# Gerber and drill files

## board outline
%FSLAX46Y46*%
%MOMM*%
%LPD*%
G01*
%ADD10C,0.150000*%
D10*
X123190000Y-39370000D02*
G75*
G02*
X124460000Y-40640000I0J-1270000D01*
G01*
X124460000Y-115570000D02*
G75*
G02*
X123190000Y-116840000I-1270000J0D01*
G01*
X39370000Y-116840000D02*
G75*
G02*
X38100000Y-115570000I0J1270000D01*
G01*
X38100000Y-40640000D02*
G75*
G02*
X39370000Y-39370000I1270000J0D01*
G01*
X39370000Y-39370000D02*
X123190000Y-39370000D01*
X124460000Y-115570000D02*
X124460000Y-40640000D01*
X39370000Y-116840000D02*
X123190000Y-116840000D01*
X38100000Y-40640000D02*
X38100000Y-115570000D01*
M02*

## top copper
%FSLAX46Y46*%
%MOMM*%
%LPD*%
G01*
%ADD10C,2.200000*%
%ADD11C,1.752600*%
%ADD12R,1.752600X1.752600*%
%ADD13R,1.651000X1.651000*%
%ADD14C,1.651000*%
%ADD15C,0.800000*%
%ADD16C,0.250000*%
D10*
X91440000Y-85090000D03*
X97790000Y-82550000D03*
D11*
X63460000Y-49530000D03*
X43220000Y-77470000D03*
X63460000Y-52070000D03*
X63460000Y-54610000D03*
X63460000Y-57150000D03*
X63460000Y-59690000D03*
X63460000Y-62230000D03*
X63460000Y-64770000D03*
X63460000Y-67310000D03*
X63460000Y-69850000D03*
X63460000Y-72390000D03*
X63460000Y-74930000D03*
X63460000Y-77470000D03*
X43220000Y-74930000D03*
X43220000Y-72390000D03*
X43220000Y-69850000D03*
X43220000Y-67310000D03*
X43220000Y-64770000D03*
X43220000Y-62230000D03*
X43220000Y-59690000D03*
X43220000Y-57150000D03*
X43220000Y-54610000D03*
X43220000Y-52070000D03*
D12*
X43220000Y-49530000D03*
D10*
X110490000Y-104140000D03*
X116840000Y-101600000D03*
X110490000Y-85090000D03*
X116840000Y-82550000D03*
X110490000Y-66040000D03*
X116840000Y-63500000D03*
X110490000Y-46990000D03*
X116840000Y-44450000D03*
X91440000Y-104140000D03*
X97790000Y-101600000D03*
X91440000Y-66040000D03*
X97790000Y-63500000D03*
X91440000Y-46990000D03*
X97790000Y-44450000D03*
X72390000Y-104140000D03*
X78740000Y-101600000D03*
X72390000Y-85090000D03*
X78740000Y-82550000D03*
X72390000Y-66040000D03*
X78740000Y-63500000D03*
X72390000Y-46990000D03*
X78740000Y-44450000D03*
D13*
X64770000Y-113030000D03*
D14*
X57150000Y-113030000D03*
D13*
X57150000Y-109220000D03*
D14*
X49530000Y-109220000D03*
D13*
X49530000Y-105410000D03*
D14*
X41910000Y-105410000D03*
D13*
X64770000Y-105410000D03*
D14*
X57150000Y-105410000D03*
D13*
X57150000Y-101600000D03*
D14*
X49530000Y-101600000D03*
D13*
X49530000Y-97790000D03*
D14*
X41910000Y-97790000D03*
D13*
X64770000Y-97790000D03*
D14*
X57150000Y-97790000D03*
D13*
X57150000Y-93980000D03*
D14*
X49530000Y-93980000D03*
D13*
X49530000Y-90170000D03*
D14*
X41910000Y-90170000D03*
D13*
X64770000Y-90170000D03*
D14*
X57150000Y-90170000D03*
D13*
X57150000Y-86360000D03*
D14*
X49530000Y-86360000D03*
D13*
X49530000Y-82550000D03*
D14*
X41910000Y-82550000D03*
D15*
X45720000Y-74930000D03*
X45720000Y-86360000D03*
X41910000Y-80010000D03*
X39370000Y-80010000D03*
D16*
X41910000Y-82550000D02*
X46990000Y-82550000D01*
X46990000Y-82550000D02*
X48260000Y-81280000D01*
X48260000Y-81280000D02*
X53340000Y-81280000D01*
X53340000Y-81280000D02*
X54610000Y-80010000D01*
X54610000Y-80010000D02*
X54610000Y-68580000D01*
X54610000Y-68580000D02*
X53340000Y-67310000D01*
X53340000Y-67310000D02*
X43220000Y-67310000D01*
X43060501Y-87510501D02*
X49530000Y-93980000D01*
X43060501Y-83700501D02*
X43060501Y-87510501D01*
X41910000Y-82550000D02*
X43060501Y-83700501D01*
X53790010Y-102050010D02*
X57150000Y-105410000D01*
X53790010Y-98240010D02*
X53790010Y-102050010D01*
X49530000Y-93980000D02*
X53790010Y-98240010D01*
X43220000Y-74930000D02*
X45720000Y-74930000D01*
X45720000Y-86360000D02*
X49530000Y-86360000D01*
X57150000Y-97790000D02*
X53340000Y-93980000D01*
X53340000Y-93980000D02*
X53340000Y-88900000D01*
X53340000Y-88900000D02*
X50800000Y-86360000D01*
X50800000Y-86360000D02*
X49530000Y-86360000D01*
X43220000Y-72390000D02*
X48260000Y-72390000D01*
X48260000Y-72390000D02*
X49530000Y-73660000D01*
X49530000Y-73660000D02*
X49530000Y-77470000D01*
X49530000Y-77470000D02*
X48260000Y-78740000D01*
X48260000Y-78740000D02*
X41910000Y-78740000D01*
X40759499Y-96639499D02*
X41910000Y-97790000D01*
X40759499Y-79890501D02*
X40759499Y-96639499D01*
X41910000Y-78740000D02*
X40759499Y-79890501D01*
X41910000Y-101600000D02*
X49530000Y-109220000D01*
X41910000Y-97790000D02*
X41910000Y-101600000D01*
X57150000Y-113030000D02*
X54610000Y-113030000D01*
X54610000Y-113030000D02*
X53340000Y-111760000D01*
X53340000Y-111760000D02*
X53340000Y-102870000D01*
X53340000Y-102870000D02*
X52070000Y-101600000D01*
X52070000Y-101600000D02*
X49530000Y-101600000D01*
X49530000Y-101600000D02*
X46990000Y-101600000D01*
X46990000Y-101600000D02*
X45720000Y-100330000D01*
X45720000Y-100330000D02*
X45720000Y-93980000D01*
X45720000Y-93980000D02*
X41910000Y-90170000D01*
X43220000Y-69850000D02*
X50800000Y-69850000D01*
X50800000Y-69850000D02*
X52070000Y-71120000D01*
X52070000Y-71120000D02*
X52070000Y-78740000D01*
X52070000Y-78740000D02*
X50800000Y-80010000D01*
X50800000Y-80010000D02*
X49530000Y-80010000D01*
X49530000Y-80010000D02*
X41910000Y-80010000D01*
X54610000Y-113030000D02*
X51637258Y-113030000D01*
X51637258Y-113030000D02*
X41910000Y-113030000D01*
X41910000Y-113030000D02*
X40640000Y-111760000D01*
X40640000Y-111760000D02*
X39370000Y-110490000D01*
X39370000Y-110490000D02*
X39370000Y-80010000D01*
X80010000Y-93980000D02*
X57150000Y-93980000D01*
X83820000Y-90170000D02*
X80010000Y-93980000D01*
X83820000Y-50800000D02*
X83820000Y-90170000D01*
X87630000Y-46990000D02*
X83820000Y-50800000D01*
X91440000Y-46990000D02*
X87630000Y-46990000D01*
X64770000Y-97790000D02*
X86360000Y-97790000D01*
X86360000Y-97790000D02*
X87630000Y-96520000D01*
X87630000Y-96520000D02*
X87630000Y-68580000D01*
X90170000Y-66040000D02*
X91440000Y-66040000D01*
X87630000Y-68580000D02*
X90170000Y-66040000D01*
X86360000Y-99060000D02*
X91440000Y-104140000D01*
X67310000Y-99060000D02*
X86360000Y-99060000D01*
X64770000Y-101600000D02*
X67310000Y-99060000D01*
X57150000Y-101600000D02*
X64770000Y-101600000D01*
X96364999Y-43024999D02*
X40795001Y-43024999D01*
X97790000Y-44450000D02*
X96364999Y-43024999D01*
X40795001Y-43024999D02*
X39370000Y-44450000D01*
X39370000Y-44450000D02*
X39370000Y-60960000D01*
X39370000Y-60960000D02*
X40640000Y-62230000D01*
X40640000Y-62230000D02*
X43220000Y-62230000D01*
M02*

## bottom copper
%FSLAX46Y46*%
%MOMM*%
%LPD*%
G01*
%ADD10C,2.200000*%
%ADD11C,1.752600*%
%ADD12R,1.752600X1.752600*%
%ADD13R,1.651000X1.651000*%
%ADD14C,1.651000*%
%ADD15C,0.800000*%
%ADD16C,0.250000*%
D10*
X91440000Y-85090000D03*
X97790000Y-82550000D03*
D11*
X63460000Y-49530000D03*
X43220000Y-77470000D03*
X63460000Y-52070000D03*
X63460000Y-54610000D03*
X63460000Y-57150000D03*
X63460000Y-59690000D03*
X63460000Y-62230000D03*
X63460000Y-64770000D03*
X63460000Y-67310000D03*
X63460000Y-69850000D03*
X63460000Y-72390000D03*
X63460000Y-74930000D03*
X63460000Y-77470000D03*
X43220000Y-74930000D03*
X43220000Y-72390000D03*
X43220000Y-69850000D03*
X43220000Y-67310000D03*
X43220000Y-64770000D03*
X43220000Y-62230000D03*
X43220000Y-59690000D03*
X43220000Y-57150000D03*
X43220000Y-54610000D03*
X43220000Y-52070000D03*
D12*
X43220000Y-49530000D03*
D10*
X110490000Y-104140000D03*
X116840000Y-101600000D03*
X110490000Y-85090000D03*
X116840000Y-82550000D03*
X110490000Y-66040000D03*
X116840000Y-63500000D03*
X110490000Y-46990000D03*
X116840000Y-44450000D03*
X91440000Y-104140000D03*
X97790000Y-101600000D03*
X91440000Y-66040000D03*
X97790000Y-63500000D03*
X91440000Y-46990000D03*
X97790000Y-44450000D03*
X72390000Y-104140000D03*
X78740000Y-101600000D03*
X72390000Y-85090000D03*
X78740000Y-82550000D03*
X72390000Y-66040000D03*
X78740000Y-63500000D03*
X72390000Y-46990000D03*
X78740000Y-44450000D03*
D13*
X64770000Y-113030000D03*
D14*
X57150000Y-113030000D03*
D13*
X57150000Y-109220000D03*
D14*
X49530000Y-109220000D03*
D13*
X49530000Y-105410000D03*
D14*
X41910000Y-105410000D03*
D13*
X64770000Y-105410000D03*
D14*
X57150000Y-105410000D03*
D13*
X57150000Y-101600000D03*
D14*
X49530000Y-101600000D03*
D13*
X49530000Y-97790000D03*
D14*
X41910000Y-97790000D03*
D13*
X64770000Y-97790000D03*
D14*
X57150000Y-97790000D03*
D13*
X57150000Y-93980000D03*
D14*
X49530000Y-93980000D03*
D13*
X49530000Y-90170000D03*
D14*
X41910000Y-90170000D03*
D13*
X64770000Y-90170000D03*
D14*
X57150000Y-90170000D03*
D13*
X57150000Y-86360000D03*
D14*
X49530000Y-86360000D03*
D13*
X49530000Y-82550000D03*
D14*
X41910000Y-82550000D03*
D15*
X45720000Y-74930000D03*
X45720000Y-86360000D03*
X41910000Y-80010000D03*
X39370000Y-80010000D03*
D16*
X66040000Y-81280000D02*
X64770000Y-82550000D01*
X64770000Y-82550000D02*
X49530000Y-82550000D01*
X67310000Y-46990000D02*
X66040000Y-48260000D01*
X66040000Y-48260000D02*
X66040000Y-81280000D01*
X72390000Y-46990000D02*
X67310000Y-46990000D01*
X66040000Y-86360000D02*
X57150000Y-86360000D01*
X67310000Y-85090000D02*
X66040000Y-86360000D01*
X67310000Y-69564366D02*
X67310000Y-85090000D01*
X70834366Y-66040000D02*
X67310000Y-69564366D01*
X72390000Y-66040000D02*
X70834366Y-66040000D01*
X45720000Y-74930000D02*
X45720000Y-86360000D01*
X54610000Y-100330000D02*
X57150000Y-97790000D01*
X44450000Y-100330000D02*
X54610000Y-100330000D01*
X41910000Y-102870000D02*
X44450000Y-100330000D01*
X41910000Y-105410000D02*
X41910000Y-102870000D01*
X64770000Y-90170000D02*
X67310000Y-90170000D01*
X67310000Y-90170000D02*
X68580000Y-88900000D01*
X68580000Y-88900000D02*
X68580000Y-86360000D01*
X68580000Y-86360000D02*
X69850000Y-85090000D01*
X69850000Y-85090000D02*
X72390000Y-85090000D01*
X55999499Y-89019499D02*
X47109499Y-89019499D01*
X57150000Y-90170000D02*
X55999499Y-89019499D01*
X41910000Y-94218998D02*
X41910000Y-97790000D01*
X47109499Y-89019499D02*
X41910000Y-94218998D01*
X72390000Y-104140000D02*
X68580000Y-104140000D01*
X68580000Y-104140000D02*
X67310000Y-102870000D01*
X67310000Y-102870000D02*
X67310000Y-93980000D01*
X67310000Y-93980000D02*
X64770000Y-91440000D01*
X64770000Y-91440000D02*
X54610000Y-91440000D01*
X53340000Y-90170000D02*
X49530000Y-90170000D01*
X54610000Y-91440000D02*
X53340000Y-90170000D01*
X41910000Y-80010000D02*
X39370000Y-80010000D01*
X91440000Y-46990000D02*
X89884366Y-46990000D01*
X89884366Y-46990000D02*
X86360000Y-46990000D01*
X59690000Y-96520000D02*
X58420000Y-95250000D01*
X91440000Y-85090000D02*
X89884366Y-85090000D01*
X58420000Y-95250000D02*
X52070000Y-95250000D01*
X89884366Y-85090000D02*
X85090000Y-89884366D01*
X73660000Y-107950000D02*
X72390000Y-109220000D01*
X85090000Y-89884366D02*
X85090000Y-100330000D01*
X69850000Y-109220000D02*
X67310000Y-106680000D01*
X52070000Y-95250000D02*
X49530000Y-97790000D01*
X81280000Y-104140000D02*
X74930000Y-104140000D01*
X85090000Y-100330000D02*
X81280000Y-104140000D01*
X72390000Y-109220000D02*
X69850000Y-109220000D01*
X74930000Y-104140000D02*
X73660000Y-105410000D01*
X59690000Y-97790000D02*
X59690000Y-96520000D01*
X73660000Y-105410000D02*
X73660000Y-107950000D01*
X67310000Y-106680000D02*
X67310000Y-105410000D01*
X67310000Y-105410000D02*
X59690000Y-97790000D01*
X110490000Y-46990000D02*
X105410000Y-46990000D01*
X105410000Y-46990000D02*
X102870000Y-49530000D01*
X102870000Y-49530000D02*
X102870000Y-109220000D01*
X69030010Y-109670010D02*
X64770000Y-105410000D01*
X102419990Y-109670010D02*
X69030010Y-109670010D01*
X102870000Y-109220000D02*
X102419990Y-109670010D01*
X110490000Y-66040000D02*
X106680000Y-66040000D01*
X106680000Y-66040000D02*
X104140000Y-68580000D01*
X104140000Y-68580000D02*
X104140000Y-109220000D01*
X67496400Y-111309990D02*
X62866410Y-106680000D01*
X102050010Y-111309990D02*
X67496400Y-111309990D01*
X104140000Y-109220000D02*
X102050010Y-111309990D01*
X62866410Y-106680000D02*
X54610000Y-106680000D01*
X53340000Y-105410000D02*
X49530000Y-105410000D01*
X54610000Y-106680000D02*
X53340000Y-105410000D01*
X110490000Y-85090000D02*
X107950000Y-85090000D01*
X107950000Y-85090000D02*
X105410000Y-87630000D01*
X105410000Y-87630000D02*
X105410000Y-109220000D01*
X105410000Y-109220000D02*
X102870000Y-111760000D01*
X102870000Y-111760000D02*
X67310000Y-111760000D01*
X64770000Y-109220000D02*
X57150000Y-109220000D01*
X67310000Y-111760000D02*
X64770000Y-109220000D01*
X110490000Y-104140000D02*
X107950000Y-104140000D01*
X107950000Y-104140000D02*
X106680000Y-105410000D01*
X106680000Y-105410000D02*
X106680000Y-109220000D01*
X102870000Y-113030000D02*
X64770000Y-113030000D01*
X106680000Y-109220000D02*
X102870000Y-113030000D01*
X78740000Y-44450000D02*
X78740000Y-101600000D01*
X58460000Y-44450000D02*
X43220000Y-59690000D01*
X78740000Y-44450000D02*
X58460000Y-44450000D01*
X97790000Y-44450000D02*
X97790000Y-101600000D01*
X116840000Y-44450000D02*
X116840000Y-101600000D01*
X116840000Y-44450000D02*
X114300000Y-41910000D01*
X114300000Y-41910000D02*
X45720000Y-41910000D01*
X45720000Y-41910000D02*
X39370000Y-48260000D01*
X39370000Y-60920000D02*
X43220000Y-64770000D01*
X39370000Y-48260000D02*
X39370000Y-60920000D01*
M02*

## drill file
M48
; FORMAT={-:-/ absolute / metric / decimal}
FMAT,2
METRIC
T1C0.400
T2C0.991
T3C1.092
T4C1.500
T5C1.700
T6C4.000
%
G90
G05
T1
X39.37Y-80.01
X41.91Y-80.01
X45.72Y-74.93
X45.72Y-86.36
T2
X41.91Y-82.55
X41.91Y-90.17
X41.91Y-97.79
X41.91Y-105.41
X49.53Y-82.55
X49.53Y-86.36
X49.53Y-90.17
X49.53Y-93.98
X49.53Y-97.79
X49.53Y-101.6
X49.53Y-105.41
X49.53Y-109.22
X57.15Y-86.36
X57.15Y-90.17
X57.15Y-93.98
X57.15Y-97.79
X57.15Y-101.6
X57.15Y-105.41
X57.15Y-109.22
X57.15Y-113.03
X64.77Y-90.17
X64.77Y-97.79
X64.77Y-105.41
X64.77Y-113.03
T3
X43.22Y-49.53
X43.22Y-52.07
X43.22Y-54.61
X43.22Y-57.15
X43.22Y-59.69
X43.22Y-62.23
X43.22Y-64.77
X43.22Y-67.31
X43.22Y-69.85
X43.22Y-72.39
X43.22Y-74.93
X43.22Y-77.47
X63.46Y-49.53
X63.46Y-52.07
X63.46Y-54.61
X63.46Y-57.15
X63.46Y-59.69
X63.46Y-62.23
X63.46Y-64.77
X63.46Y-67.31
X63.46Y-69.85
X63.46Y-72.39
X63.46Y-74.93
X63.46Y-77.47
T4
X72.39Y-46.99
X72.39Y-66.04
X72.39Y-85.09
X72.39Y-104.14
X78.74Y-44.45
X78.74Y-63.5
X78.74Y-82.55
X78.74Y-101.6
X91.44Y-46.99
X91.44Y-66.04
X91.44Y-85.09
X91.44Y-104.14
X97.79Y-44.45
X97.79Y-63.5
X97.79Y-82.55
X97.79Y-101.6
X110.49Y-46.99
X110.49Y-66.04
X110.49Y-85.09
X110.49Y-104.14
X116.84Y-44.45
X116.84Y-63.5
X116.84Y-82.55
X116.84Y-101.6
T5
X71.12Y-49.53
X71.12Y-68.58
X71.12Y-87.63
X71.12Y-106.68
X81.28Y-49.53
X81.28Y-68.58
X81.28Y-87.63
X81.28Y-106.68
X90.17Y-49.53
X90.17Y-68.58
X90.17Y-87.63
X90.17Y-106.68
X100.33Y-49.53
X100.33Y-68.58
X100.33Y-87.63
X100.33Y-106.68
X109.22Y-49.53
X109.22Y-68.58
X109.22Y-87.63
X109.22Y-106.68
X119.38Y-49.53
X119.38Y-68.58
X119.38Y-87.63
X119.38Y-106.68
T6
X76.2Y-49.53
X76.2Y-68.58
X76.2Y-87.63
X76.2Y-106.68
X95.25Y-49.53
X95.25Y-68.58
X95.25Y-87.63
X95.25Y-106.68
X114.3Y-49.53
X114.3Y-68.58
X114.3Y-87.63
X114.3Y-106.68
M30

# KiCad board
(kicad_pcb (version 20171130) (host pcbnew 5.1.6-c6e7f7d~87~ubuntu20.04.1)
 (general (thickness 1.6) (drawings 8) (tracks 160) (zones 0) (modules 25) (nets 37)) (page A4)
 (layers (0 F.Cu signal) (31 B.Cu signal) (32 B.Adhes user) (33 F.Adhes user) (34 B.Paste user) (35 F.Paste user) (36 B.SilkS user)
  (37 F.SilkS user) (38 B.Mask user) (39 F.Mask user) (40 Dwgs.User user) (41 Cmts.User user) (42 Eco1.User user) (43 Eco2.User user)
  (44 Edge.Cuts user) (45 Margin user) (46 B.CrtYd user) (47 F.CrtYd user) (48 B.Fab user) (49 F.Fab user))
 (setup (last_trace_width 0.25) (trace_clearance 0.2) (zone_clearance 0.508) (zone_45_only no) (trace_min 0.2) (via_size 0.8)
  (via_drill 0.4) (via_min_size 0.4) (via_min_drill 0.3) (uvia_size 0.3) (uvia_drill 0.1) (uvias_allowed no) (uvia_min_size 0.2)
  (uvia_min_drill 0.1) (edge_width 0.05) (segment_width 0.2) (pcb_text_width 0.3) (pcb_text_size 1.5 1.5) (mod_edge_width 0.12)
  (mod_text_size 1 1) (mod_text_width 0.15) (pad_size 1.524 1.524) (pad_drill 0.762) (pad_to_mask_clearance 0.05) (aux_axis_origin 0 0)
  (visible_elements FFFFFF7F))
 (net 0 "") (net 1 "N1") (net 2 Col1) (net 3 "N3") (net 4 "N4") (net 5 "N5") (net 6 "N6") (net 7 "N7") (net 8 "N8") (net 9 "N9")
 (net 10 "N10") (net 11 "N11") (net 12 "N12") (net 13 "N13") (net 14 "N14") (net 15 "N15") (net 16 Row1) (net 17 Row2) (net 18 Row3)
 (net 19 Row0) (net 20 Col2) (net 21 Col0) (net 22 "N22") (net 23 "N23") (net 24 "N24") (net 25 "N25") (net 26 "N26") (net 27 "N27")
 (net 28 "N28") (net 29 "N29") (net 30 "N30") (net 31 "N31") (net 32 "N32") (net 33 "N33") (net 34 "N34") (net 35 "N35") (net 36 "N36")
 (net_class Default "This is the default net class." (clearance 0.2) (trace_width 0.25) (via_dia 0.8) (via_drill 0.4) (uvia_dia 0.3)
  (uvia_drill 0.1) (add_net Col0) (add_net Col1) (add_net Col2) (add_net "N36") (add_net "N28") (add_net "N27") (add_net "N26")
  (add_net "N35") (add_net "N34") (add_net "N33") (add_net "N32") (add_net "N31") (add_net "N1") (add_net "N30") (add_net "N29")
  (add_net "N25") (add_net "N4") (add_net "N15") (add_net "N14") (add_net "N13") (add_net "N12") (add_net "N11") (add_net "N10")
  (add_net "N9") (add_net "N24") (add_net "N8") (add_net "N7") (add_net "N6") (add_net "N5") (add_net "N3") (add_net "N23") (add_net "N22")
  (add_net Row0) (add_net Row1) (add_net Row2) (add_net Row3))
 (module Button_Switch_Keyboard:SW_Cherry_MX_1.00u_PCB (layer F.Cu) (at 97.79 82.55)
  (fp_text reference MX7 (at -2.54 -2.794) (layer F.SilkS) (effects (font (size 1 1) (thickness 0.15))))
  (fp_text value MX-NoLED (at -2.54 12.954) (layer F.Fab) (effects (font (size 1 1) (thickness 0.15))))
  (pad "" np_thru_hole circle (at 2.54 5.08) (size 1.7 1.7) (drill 1.7) (layers *.Cu *.Mask))
  (pad "" np_thru_hole circle (at -7.62 5.08) (size 1.7 1.7) (drill 1.7) (layers *.Cu *.Mask))
  (pad "" np_thru_hole circle (at -2.54 5.08) (size 4 4) (drill 4) (layers *.Cu *.Mask))
  (pad 2 thru_hole circle (at -6.35 2.54) (size 2.2 2.2) (drill 1.5) (layers *.Cu *.Mask) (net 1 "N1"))
  (pad 1 thru_hole circle (at 0 0) (size 2.2 2.2) (drill 1.5) (layers *.Cu *.Mask) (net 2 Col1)))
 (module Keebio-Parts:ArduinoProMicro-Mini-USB (layer F.Cu) (at 53.34 63.5 270)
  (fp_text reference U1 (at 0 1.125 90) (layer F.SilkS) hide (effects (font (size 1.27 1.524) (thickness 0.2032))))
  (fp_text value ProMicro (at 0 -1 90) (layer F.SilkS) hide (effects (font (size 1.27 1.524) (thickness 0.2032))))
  (pad 24 thru_hole circle (at -13.97 -10.12 270) (size 1.7526 1.7526) (drill 1.0922) (layers *.Cu *.SilkS *.Mask) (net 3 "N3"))
  (pad 12 thru_hole circle (at 13.97 10.12 270) (size 1.7526 1.7526) (drill 1.0922) (layers *.Cu *.SilkS *.Mask) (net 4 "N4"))
  (pad 23 thru_hole circle (at -11.43 -10.12 270) (size 1.7526 1.7526) (drill 1.0922) (layers *.Cu *.SilkS *.Mask) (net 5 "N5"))
  (pad 22 thru_hole circle (at -8.89 -10.12 270) (size 1.7526 1.7526) (drill 1.0922) (layers *.Cu *.SilkS *.Mask) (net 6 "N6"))
  (pad 21 thru_hole circle (at -6.35 -10.12 270) (size 1.7526 1.7526) (drill 1.0922) (layers *.Cu *.SilkS *.Mask) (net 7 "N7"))
  (pad 20 thru_hole circle (at -3.81 -10.12 270) (size 1.7526 1.7526) (drill 1.0922) (layers *.Cu *.SilkS *.Mask) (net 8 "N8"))
  (pad 19 thru_hole circle (at -1.27 -10.12 270) (size 1.7526 1.7526) (drill 1.0922) (layers *.Cu *.SilkS *.Mask) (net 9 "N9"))
  (pad 18 thru_hole circle (at 1.27 -10.12 270) (size 1.7526 1.7526) (drill 1.0922) (layers *.Cu *.SilkS *.Mask) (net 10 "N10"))
  (pad 17 thru_hole circle (at 3.81 -10.12 270) (size 1.7526 1.7526) (drill 1.0922) (layers *.Cu *.SilkS *.Mask) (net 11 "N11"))
  (pad 16 thru_hole circle (at 6.35 -10.12 270) (size 1.7526 1.7526) (drill 1.0922) (layers *.Cu *.SilkS *.Mask) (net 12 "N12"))
  (pad 15 thru_hole circle (at 8.89 -10.12 270) (size 1.7526 1.7526) (drill 1.0922) (layers *.Cu *.SilkS *.Mask) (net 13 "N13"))
  (pad 14 thru_hole circle (at 11.43 -10.12 270) (size 1.7526 1.7526) (drill 1.0922) (layers *.Cu *.SilkS *.Mask) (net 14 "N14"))
  (pad 13 thru_hole circle (at 13.97 -10.12 270) (size 1.7526 1.7526) (drill 1.0922) (layers *.Cu *.SilkS *.Mask) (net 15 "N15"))
  (pad 11 thru_hole circle (at 11.43 10.12 270) (size 1.7526 1.7526) (drill 1.0922) (layers *.Cu *.SilkS *.Mask) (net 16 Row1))
  (pad 10 thru_hole circle (at 8.89 10.12 270) (size 1.7526 1.7526) (drill 1.0922) (layers *.Cu *.SilkS *.Mask) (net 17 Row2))
  (pad 9 thru_hole circle (at 6.35 10.12 270) (size 1.7526 1.7526) (drill 1.0922) (layers *.Cu *.SilkS *.Mask) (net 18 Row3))
  (pad 8 thru_hole circle (at 3.81 10.12 270) (size 1.7526 1.7526) (drill 1.0922) (layers *.Cu *.SilkS *.Mask) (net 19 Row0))
  (pad 7 thru_hole circle (at 1.27 10.12 270) (size 1.7526 1.7526) (drill 1.0922) (layers *.Cu *.SilkS *.Mask) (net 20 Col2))
  (pad 6 thru_hole circle (at -1.27 10.12 270) (size 1.7526 1.7526) (drill 1.0922) (layers *.Cu *.SilkS *.Mask) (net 2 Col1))
  (pad 5 thru_hole circle (at -3.81 10.12 270) (size 1.7526 1.7526) (drill 1.0922) (layers *.Cu *.SilkS *.Mask) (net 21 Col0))
  (pad 4 thru_hole circle (at -6.35 10.12 270) (size 1.7526 1.7526) (drill 1.0922) (layers *.Cu *.SilkS *.Mask) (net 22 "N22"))
  (pad 3 thru_hole circle (at -8.89 10.12 270) (size 1.7526 1.7526) (drill 1.0922) (layers *.Cu *.SilkS *.Mask) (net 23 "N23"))
  (pad 2 thru_hole circle (at -11.43 10.12 270) (size 1.7526 1.7526) (drill 1.0922) (layers *.Cu *.SilkS *.Mask) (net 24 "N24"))
  (pad 1 thru_hole rect (at -13.97 10.12 270) (size 1.7526 1.7526) (drill 1.0922) (layers *.Cu *.SilkS *.Mask) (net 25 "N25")))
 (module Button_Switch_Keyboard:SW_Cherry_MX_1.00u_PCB (layer F.Cu) (at 116.84 101.6)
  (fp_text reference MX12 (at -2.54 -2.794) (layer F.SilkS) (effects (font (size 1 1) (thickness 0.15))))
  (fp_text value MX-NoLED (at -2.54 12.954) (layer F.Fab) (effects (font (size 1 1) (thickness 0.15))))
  (pad "" np_thru_hole circle (at 2.54 5.08) (size 1.7 1.7) (drill 1.7) (layers *.Cu *.Mask))
  (pad "" np_thru_hole circle (at -7.62 5.08) (size 1.7 1.7) (drill 1.7) (layers *.Cu *.Mask))
  (pad "" np_thru_hole circle (at -2.54 5.08) (size 4 4) (drill 4) (layers *.Cu *.Mask))
  (pad 2 thru_hole circle (at -6.35 2.54) (size 2.2 2.2) (drill 1.5) (layers *.Cu *.Mask) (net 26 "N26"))
  (pad 1 thru_hole circle (at 0 0) (size 2.2 2.2) (drill 1.5) (layers *.Cu *.Mask) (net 20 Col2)))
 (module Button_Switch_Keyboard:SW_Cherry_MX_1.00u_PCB (layer F.Cu) (at 116.84 82.55)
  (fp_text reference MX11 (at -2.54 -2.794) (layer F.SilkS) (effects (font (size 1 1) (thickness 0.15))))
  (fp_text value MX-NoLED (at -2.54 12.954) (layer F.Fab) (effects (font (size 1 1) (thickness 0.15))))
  (pad "" np_thru_hole circle (at 2.54 5.08) (size 1.7 1.7) (drill 1.7) (layers *.Cu *.Mask))
  (pad "" np_thru_hole circle (at -7.62 5.08) (size 1.7 1.7) (drill 1.7) (layers *.Cu *.Mask))
  (pad "" np_thru_hole circle (at -2.54 5.08) (size 4 4) (drill 4) (layers *.Cu *.Mask))
  (pad 2 thru_hole circle (at -6.35 2.54) (size 2.2 2.2) (drill 1.5) (layers *.Cu *.Mask) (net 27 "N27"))
  (pad 1 thru_hole circle (at 0 0) (size 2.2 2.2) (drill 1.5) (layers *.Cu *.Mask) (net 20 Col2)))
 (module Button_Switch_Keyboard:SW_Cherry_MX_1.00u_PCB (layer F.Cu) (at 116.84 63.5)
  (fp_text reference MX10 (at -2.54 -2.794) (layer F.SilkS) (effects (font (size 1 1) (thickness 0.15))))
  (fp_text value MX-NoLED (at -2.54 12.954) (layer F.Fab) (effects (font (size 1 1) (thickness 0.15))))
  (pad "" np_thru_hole circle (at 2.54 5.08) (size 1.7 1.7) (drill 1.7) (layers *.Cu *.Mask))
  (pad "" np_thru_hole circle (at -7.62 5.08) (size 1.7 1.7) (drill 1.7) (layers *.Cu *.Mask))
  (pad "" np_thru_hole circle (at -2.54 5.08) (size 4 4) (drill 4) (layers *.Cu *.Mask))
  (pad 2 thru_hole circle (at -6.35 2.54) (size 2.2 2.2) (drill 1.5) (layers *.Cu *.Mask) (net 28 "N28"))
  (pad 1 thru_hole circle (at 0 0) (size 2.2 2.2) (drill 1.5) (layers *.Cu *.Mask) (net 20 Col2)))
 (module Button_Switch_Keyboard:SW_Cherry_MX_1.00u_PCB (layer F.Cu) (at 116.84 44.45)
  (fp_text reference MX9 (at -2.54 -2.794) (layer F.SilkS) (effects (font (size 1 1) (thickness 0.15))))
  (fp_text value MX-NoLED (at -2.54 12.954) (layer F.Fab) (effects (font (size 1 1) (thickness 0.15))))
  (pad "" np_thru_hole circle (at 2.54 5.08) (size 1.7 1.7) (drill 1.7) (layers *.Cu *.Mask))
  (pad "" np_thru_hole circle (at -7.62 5.08) (size 1.7 1.7) (drill 1.7) (layers *.Cu *.Mask))
  (pad "" np_thru_hole circle (at -2.54 5.08) (size 4 4) (drill 4) (layers *.Cu *.Mask))
  (pad 2 thru_hole circle (at -6.35 2.54) (size 2.2 2.2) (drill 1.5) (layers *.Cu *.Mask) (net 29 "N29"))
  (pad 1 thru_hole circle (at 0 0) (size 2.2 2.2) (drill 1.5) (layers *.Cu *.Mask) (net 20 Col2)))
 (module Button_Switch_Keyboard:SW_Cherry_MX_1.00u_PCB (layer F.Cu) (at 97.79 101.6)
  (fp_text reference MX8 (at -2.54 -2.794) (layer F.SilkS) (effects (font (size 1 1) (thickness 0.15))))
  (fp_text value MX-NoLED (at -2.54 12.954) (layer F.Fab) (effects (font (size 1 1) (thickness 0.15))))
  (pad "" np_thru_hole circle (at 2.54 5.08) (size 1.7 1.7) (drill 1.7) (layers *.Cu *.Mask))
  (pad "" np_thru_hole circle (at -7.62 5.08) (size 1.7 1.7) (drill 1.7) (layers *.Cu *.Mask))
  (pad "" np_thru_hole circle (at -2.54 5.08) (size 4 4) (drill 4) (layers *.Cu *.Mask))
  (pad 2 thru_hole circle (at -6.35 2.54) (size 2.2 2.2) (drill 1.5) (layers *.Cu *.Mask) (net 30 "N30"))
  (pad 1 thru_hole circle (at 0 0) (size 2.2 2.2) (drill 1.5) (layers *.Cu *.Mask) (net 2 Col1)))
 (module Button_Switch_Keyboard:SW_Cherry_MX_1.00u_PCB (layer F.Cu) (at 97.79 63.5)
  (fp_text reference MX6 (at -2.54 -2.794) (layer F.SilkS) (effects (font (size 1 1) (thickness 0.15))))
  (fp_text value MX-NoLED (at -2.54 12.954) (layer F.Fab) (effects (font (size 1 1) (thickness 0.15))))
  (pad "" np_thru_hole circle (at 2.54 5.08) (size 1.7 1.7) (drill 1.7) (layers *.Cu *.Mask))
  (pad "" np_thru_hole circle (at -7.62 5.08) (size 1.7 1.7) (drill 1.7) (layers *.Cu *.Mask))
  (pad "" np_thru_hole circle (at -2.54 5.08) (size 4 4) (drill 4) (layers *.Cu *.Mask))
  (pad 2 thru_hole circle (at -6.35 2.54) (size 2.2 2.2) (drill 1.5) (layers *.Cu *.Mask) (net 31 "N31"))
  (pad 1 thru_hole circle (at 0 0) (size 2.2 2.2) (drill 1.5) (layers *.Cu *.Mask) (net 2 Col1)))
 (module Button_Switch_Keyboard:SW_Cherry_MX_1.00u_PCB (layer F.Cu) (at 97.79 44.45)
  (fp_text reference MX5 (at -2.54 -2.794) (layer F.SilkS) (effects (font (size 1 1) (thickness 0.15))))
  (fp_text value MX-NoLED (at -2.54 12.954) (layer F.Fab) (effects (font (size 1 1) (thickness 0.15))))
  (pad "" np_thru_hole circle (at 2.54 5.08) (size 1.7 1.7) (drill 1.7) (layers *.Cu *.Mask))
  (pad "" np_thru_hole circle (at -7.62 5.08) (size 1.7 1.7) (drill 1.7) (layers *.Cu *.Mask))
  (pad "" np_thru_hole circle (at -2.54 5.08) (size 4 4) (drill 4) (layers *.Cu *.Mask))
  (pad 2 thru_hole circle (at -6.35 2.54) (size 2.2 2.2) (drill 1.5) (layers *.Cu *.Mask) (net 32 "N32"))
  (pad 1 thru_hole circle (at 0 0) (size 2.2 2.2) (drill 1.5) (layers *.Cu *.Mask) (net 2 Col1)))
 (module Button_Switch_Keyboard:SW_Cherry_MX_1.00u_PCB (layer F.Cu) (at 78.74 101.6)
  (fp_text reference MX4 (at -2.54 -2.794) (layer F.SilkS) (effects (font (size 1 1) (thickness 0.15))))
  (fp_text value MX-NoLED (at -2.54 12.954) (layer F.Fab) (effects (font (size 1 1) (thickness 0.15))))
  (pad "" np_thru_hole circle (at 2.54 5.08) (size 1.7 1.7) (drill 1.7) (layers *.Cu *.Mask))
  (pad "" np_thru_hole circle (at -7.62 5.08) (size 1.7 1.7) (drill 1.7) (layers *.Cu *.Mask))
  (pad "" np_thru_hole circle (at -2.54 5.08) (size 4 4) (drill 4) (layers *.Cu *.Mask))
  (pad 2 thru_hole circle (at -6.35 2.54) (size 2.2 2.2) (drill 1.5) (layers *.Cu *.Mask) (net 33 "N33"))
  (pad 1 thru_hole circle (at 0 0) (size 2.2 2.2) (drill 1.5) (layers *.Cu *.Mask) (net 21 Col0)))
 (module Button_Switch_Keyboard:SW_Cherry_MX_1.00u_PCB (layer F.Cu) (at 78.74 82.55)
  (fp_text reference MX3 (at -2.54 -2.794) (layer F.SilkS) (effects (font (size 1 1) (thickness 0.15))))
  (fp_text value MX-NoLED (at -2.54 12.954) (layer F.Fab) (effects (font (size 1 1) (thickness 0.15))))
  (pad "" np_thru_hole circle (at 2.54 5.08) (size 1.7 1.7) (drill 1.7) (layers *.Cu *.Mask))
  (pad "" np_thru_hole circle (at -7.62 5.08) (size 1.7 1.7) (drill 1.7) (layers *.Cu *.Mask))
  (pad "" np_thru_hole circle (at -2.54 5.08) (size 4 4) (drill 4) (layers *.Cu *.Mask))
  (pad 2 thru_hole circle (at -6.35 2.54) (size 2.2 2.2) (drill 1.5) (layers *.Cu *.Mask) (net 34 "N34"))
  (pad 1 thru_hole circle (at 0 0) (size 2.2 2.2) (drill 1.5) (layers *.Cu *.Mask) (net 21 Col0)))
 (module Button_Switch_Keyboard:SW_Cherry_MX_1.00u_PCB (layer F.Cu) (at 78.74 63.5)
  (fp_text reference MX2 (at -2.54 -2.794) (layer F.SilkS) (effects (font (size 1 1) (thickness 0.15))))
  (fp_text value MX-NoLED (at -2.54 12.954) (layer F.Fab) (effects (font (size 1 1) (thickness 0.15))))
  (pad "" np_thru_hole circle (at 2.54 5.08) (size 1.7 1.7) (drill 1.7) (layers *.Cu *.Mask))
  (pad "" np_thru_hole circle (at -7.62 5.08) (size 1.7 1.7) (drill 1.7) (layers *.Cu *.Mask))
  (pad "" np_thru_hole circle (at -2.54 5.08) (size 4 4) (drill 4) (layers *.Cu *.Mask))
  (pad 2 thru_hole circle (at -6.35 2.54) (size 2.2 2.2) (drill 1.5) (layers *.Cu *.Mask) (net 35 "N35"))
  (pad 1 thru_hole circle (at 0 0) (size 2.2 2.2) (drill 1.5) (layers *.Cu *.Mask) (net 21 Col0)))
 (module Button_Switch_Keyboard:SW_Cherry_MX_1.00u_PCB (layer F.Cu) (at 78.74 44.45)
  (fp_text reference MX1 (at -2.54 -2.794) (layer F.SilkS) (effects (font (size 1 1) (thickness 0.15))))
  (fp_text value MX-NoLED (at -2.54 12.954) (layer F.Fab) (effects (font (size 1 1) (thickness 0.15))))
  (pad "" np_thru_hole circle (at 2.54 5.08) (size 1.7 1.7) (drill 1.7) (layers *.Cu *.Mask))
  (pad "" np_thru_hole circle (at -7.62 5.08) (size 1.7 1.7) (drill 1.7) (layers *.Cu *.Mask))
  (pad "" np_thru_hole circle (at -2.54 5.08) (size 4 4) (drill 4) (layers *.Cu *.Mask))
  (pad 2 thru_hole circle (at -6.35 2.54) (size 2.2 2.2) (drill 1.5) (layers *.Cu *.Mask) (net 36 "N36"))
  (pad 1 thru_hole circle (at 0 0) (size 2.2 2.2) (drill 1.5) (layers *.Cu *.Mask) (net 21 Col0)))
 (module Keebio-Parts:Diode (layer F.Cu) (at 60.96 113.03)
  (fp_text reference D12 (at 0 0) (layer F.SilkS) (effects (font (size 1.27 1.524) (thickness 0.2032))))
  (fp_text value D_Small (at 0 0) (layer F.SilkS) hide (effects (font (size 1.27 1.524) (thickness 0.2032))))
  (pad 2 thru_hole rect (at 3.81 0) (size 1.651 1.651) (drill 0.9906) (layers *.Cu *.SilkS *.Mask) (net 26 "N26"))
  (pad 1 thru_hole circle (at -3.81 0) (size 1.651 1.651) (drill 0.9906) (layers *.Cu *.SilkS *.Mask) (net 18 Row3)))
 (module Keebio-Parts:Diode (layer F.Cu) (at 53.34 109.22)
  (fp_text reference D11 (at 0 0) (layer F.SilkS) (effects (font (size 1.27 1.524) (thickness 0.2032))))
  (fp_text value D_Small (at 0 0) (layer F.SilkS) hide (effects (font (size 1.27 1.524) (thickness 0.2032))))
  (pad 2 thru_hole rect (at 3.81 0) (size 1.651 1.651) (drill 0.9906) (layers *.Cu *.SilkS *.Mask) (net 27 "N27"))
  (pad 1 thru_hole circle (at -3.81 0) (size 1.651 1.651) (drill 0.9906) (layers *.Cu *.SilkS *.Mask) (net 17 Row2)))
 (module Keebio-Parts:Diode (layer F.Cu) (at 45.72 105.41)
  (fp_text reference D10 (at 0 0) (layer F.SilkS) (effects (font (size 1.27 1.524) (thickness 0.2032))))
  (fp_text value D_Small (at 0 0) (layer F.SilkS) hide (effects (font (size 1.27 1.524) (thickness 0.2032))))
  (pad 2 thru_hole rect (at 3.81 0) (size 1.651 1.651) (drill 0.9906) (layers *.Cu *.SilkS *.Mask) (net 28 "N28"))
  (pad 1 thru_hole circle (at -3.81 0) (size 1.651 1.651) (drill 0.9906) (layers *.Cu *.SilkS *.Mask) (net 16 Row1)))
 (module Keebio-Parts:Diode (layer F.Cu) (at 60.96 105.41)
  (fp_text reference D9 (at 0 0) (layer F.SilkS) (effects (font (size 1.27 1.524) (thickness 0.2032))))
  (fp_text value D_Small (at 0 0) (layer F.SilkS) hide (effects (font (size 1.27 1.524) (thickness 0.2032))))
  (pad 2 thru_hole rect (at 3.81 0) (size 1.651 1.651) (drill 0.9906) (layers *.Cu *.SilkS *.Mask) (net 29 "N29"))
  (pad 1 thru_hole circle (at -3.81 0) (size 1.651 1.651) (drill 0.9906) (layers *.Cu *.SilkS *.Mask) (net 19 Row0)))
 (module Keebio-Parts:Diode (layer F.Cu) (at 53.34 101.6)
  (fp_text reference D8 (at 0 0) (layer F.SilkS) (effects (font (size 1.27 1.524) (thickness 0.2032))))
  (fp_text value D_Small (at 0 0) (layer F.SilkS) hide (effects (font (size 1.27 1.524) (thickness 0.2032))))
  (pad 2 thru_hole rect (at 3.81 0) (size 1.651 1.651) (drill 0.9906) (layers *.Cu *.SilkS *.Mask) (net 30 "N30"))
  (pad 1 thru_hole circle (at -3.81 0) (size 1.651 1.651) (drill 0.9906) (layers *.Cu *.SilkS *.Mask) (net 18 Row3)))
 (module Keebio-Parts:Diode (layer F.Cu) (at 45.72 97.79)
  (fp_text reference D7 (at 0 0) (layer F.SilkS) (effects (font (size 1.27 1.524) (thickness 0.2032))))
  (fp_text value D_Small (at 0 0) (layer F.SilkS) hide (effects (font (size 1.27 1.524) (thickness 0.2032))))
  (pad 2 thru_hole rect (at 3.81 0) (size 1.651 1.651) (drill 0.9906) (layers *.Cu *.SilkS *.Mask) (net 1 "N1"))
  (pad 1 thru_hole circle (at -3.81 0) (size 1.651 1.651) (drill 0.9906) (layers *.Cu *.SilkS *.Mask) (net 17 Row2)))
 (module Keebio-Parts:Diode (layer F.Cu) (at 60.96 97.79)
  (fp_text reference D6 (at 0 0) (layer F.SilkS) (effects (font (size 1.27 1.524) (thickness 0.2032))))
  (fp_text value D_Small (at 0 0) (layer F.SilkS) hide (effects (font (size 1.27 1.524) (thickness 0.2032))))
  (pad 2 thru_hole rect (at 3.81 0) (size 1.651 1.651) (drill 0.9906) (layers *.Cu *.SilkS *.Mask) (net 31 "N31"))
  (pad 1 thru_hole circle (at -3.81 0) (size 1.651 1.651) (drill 0.9906) (layers *.Cu *.SilkS *.Mask) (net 16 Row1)))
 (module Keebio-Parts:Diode (layer F.Cu) (at 53.34 93.98)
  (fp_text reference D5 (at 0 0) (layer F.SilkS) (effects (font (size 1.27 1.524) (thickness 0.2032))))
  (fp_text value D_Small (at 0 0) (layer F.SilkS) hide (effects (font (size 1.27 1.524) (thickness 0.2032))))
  (pad 2 thru_hole rect (at 3.81 0) (size 1.651 1.651) (drill 0.9906) (layers *.Cu *.SilkS *.Mask) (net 32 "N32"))
  (pad 1 thru_hole circle (at -3.81 0) (size 1.651 1.651) (drill 0.9906) (layers *.Cu *.SilkS *.Mask) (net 19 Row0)))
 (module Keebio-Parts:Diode (layer F.Cu) (at 45.72 90.17)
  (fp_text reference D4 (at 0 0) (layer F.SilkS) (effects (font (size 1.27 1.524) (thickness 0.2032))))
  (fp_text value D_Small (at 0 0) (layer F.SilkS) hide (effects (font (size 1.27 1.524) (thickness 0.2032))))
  (pad 2 thru_hole rect (at 3.81 0) (size 1.651 1.651) (drill 0.9906) (layers *.Cu *.SilkS *.Mask) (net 33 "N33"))
  (pad 1 thru_hole circle (at -3.81 0) (size 1.651 1.651) (drill 0.9906) (layers *.Cu *.SilkS *.Mask) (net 18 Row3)))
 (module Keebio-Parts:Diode (layer F.Cu) (at 60.96 90.17)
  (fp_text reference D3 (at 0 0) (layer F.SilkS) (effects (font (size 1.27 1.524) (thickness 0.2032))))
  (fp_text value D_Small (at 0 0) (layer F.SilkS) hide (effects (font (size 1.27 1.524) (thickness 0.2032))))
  (pad 2 thru_hole rect (at 3.81 0) (size 1.651 1.651) (drill 0.9906) (layers *.Cu *.SilkS *.Mask) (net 34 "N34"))
  (pad 1 thru_hole circle (at -3.81 0) (size 1.651 1.651) (drill 0.9906) (layers *.Cu *.SilkS *.Mask) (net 17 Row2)))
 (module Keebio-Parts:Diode (layer F.Cu) (at 53.34 86.36)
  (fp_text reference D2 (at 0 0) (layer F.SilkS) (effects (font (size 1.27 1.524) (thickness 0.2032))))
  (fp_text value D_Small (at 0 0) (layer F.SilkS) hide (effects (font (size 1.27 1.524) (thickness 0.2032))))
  (pad 2 thru_hole rect (at 3.81 0) (size 1.651 1.651) (drill 0.9906) (layers *.Cu *.SilkS *.Mask) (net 35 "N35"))
  (pad 1 thru_hole circle (at -3.81 0) (size 1.651 1.651) (drill 0.9906) (layers *.Cu *.SilkS *.Mask) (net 16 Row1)))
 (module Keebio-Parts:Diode (layer F.Cu) (at 45.72 82.55)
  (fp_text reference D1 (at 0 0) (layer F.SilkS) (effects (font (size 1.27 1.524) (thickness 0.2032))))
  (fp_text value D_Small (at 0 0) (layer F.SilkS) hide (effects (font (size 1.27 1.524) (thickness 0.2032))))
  (pad 2 thru_hole rect (at 3.81 0) (size 1.651 1.651) (drill 0.9906) (layers *.Cu *.SilkS *.Mask) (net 36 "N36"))
  (pad 1 thru_hole circle (at -3.81 0) (size 1.651 1.651) (drill 0.9906) (layers *.Cu *.SilkS *.Mask) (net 19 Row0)))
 (gr_arc (start 123.19 40.64) (end 124.46 40.64) (angle -90) (layer Edge.Cuts) (width 0.15))
 (gr_arc (start 123.19 115.57) (end 123.19 116.84) (angle -90) (layer Edge.Cuts) (width 0.15))
 (gr_arc (start 39.37 115.57) (end 38.1 115.57) (angle -90) (layer Edge.Cuts) (width 0.15))
 (gr_arc (start 39.37 40.64) (end 39.37 39.37) (angle -90) (layer Edge.Cuts) (width 0.15))
 (gr_line (start 39.37 39.37) (end 123.19 39.37) (layer Edge.Cuts) (width 0.15))
 (gr_line (start 124.46 115.57) (end 124.46 40.64) (layer Edge.Cuts) (width 0.15))
 (gr_line (start 39.37 116.84) (end 123.19 116.84) (layer Edge.Cuts) (width 0.15))
 (gr_line (start 38.1 40.64) (end 38.1 115.57) (layer Edge.Cuts) (width 0.15))
 (segment (start 66.04 81.28) (end 64.77 82.55) (width 0.25) (layer B.Cu) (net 36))
 (segment (start 64.77 82.55) (end 49.53 82.55) (width 0.25) (layer B.Cu) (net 36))
 (segment (start 67.31 46.99) (end 66.04 48.26) (width 0.25) (layer B.Cu) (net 36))
 (segment (start 66.04 48.26) (end 66.04 81.28) (width 0.25) (layer B.Cu) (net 36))
 (segment (start 72.39 46.99) (end 67.31 46.99) (width 0.25) (layer B.Cu) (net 36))
 (segment (start 41.91 82.55) (end 46.99 82.55) (width 0.25) (layer F.Cu) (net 19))
 (segment (start 46.99 82.55) (end 48.26 81.28) (width 0.25) (layer F.Cu) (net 19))
 (segment (start 48.26 81.28) (end 53.34 81.28) (width 0.25) (layer F.Cu) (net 19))
 (segment (start 53.34 81.28) (end 54.61 80.01) (width 0.25) (layer F.Cu) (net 19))
 (segment (start 54.61 80.01) (end 54.61 68.58) (width 0.25) (layer F.Cu) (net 19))
 (segment (start 54.61 68.58) (end 53.34 67.31) (width 0.25) (layer F.Cu) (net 19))
 (segment (start 53.34 67.31) (end 43.22 67.31) (width 0.25) (layer F.Cu) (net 19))
 (segment (start 43.060501 87.510501) (end 49.53 93.98) (width 0.25) (layer F.Cu) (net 19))
 (segment (start 43.060501 83.700501) (end 43.060501 87.510501) (width 0.25) (layer F.Cu) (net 19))
 (segment (start 41.91 82.55) (end 43.060501 83.700501) (width 0.25) (layer F.Cu) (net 19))
 (segment (start 53.79001 102.05001) (end 57.15 105.41) (width 0.25) (layer F.Cu) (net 19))
 (segment (start 53.79001 98.24001) (end 53.79001 102.05001) (width 0.25) (layer F.Cu) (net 19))
 (segment (start 49.53 93.98) (end 53.79001 98.24001) (width 0.25) (layer F.Cu) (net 19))
 (segment (start 66.04 86.36) (end 57.15 86.36) (width 0.25) (layer B.Cu) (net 35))
 (segment (start 67.31 85.09) (end 66.04 86.36) (width 0.25) (layer B.Cu) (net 35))
 (segment (start 67.31 69.564366) (end 67.31 85.09) (width 0.25) (layer B.Cu) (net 35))
 (segment (start 70.834366 66.04) (end 67.31 69.564366) (width 0.25) (layer B.Cu) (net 35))
 (segment (start 72.39 66.04) (end 70.834366 66.04) (width 0.25) (layer B.Cu) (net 35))
 (segment (start 43.22 74.93) (end 45.72 74.93) (width 0.25) (layer F.Cu) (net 16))
 (via (at 45.72 74.93) (size 0.8) (drill 0.4) (layers F.Cu B.Cu) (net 16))
 (via (at 45.72 86.36) (size 0.8) (drill 0.4) (layers F.Cu B.Cu) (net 16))
 (segment (start 45.72 74.93) (end 45.72 86.36) (width 0.25) (layer B.Cu) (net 16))
 (segment (start 45.72 86.36) (end 49.53 86.36) (width 0.25) (layer F.Cu) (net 16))
 (segment (start 54.61 100.33) (end 57.15 97.79) (width 0.25) (layer B.Cu) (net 16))
 (segment (start 44.45 100.33) (end 54.61 100.33) (width 0.25) (layer B.Cu) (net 16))
 (segment (start 41.91 102.87) (end 44.45 100.33) (width 0.25) (layer B.Cu) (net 16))
 (segment (start 41.91 105.41) (end 41.91 102.87) (width 0.25) (layer B.Cu) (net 16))
 (segment (start 57.15 97.79) (end 53.34 93.98) (width 0.25) (layer F.Cu) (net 16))
 (segment (start 53.34 93.98) (end 53.34 88.9) (width 0.25) (layer F.Cu) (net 16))
 (segment (start 53.34 88.9) (end 50.8 86.36) (width 0.25) (layer F.Cu) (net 16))
 (segment (start 50.8 86.36) (end 49.53 86.36) (width 0.25) (layer F.Cu) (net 16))
 (segment (start 64.77 90.17) (end 67.31 90.17) (width 0.25) (layer B.Cu) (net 34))
 (segment (start 67.31 90.17) (end 68.58 88.9) (width 0.25) (layer B.Cu) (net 34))
 (segment (start 68.58 88.9) (end 68.58 86.36) (width 0.25) (layer B.Cu) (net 34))
 (segment (start 68.58 86.36) (end 69.85 85.09) (width 0.25) (layer B.Cu) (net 34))
 (segment (start 69.85 85.09) (end 72.39 85.09) (width 0.25) (layer B.Cu) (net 34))
 (segment (start 43.22 72.39) (end 48.26 72.39) (width 0.25) (layer F.Cu) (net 17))
 (segment (start 48.26 72.39) (end 49.53 73.66) (width 0.25) (layer F.Cu) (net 17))
 (segment (start 49.53 73.66) (end 49.53 77.47) (width 0.25) (layer F.Cu) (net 17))
 (segment (start 49.53 77.47) (end 48.26 78.74) (width 0.25) (layer F.Cu) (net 17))
 (segment (start 48.26 78.74) (end 41.91 78.74) (width 0.25) (layer F.Cu) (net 17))
 (segment (start 40.759499 96.639499) (end 41.91 97.79) (width 0.25) (layer F.Cu) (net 17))
 (segment (start 40.759499 79.890501) (end 40.759499 96.639499) (width 0.25) (layer F.Cu) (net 17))
 (segment (start 41.91 78.74) (end 40.759499 79.890501) (width 0.25) (layer F.Cu) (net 17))
 (segment (start 55.999499 89.019499) (end 47.109499 89.019499) (width 0.25) (layer B.Cu) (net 17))
 (segment (start 57.15 90.17) (end 55.999499 89.019499) (width 0.25) (layer B.Cu) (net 17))
 (segment (start 41.91 94.218998) (end 41.91 97.79) (width 0.25) (layer B.Cu) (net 17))
 (segment (start 47.109499 89.019499) (end 41.91 94.218998) (width 0.25) (layer B.Cu) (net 17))
 (segment (start 41.91 101.6) (end 49.53 109.22) (width 0.25) (layer F.Cu) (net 17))
 (segment (start 41.91 97.79) (end 41.91 101.6) (width 0.25) (layer F.Cu) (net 17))
 (segment (start 72.39 104.14) (end 68.58 104.14) (width 0.25) (layer B.Cu) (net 33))
 (segment (start 68.58 104.14) (end 67.31 102.87) (width 0.25) (layer B.Cu) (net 33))
 (segment (start 67.31 102.87) (end 67.31 93.98) (width 0.25) (layer B.Cu) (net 33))
 (segment (start 67.31 93.98) (end 64.77 91.44) (width 0.25) (layer B.Cu) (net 33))
 (segment (start 64.77 91.44) (end 54.61 91.44) (width 0.25) (layer B.Cu) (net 33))
 (segment (start 53.34 90.17) (end 49.53 90.17) (width 0.25) (layer B.Cu) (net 33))
 (segment (start 54.61 91.44) (end 53.34 90.17) (width 0.25) (layer B.Cu) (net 33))
 (segment (start 57.15 113.03) (end 54.61 113.03) (width 0.25) (layer F.Cu) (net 18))
 (segment (start 54.61 113.03) (end 53.34 111.76) (width 0.25) (layer F.Cu) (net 18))
 (segment (start 53.34 111.76) (end 53.34 102.87) (width 0.25) (layer F.Cu) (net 18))
 (segment (start 53.34 102.87) (end 52.07 101.6) (width 0.25) (layer F.Cu) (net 18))
 (segment (start 52.07 101.6) (end 49.53 101.6) (width 0.25) (layer F.Cu) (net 18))
 (segment (start 49.53 101.6) (end 46.99 101.6) (width 0.25) (layer F.Cu) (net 18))
 (segment (start 46.99 101.6) (end 45.72 100.33) (width 0.25) (layer F.Cu) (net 18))
 (segment (start 45.72 100.33) (end 45.72 93.98) (width 0.25) (layer F.Cu) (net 18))
 (segment (start 45.72 93.98) (end 41.91 90.17) (width 0.25) (layer F.Cu) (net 18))
 (segment (start 43.22 69.85) (end 50.8 69.85) (width 0.25) (layer F.Cu) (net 18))
 (segment (start 50.8 69.85) (end 52.07 71.12) (width 0.25) (layer F.Cu) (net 18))
 (segment (start 52.07 71.12) (end 52.07 78.74) (width 0.25) (layer F.Cu) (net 18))
 (segment (start 52.07 78.74) (end 50.8 80.01) (width 0.25) (layer F.Cu) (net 18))
 (segment (start 50.8 80.01) (end 49.53 80.01) (width 0.25) (layer F.Cu) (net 18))
 (segment (start 49.53 80.01) (end 41.91 80.01) (width 0.25) (layer F.Cu) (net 18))
 (via (at 41.91 80.01) (size 0.8) (drill 0.4) (layers F.Cu B.Cu) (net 18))
 (segment (start 54.61 113.03) (end 51.637258 113.03) (width 0.25) (layer F.Cu) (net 18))
 (segment (start 51.637258 113.03) (end 41.91 113.03) (width 0.25) (layer F.Cu) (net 18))
 (segment (start 41.91 113.03) (end 40.64 111.76) (width 0.25) (layer F.Cu) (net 18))
 (segment (start 40.64 111.76) (end 39.37 110.49) (width 0.25) (layer F.Cu) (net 18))
 (via (at 39.37 80.01) (size 0.8) (drill 0.4) (layers F.Cu B.Cu) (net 18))
 (segment (start 39.37 110.49) (end 39.37 80.01) (width 0.25) (layer F.Cu) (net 18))
 (segment (start 41.91 80.01) (end 39.37 80.01) (width 0.25) (layer B.Cu) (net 18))
 (segment (start 91.44 46.99) (end 89.884366 46.99) (width 0.25) (layer B.Cu) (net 32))
 (segment (start 89.884366 46.99) (end 86.36 46.99) (width 0.25) (layer B.Cu) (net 32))
 (segment (start 80.01 93.98) (end 57.15 93.98) (width 0.25) (layer F.Cu) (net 32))
 (segment (start 83.82 90.17) (end 80.01 93.98) (width 0.25) (layer F.Cu) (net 32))
 (segment (start 83.82 50.8) (end 83.82 90.17) (width 0.25) (layer F.Cu) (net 32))
 (segment (start 87.63 46.99) (end 83.82 50.8) (width 0.25) (layer F.Cu) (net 32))
 (segment (start 91.44 46.99) (end 87.63 46.99) (width 0.25) (layer F.Cu) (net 32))
 (segment (start 64.77 97.79) (end 86.36 97.79) (width 0.25) (layer F.Cu) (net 31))
 (segment (start 86.36 97.79) (end 87.63 96.52) (width 0.25) (layer F.Cu) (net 31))
 (segment (start 87.63 96.52) (end 87.63 68.58) (width 0.25) (layer F.Cu) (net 31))
 (segment (start 90.17 66.04) (end 91.44 66.04) (width 0.25) (layer F.Cu) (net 31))
 (segment (start 87.63 68.58) (end 90.17 66.04) (width 0.25) (layer F.Cu) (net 31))
 (segment (start 59.69 96.52) (end 58.42 95.25) (width 0.25) (layer B.Cu) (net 1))
 (segment (start 91.44 85.09) (end 89.884366 85.09) (width 0.25) (layer B.Cu) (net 1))
 (segment (start 58.42 95.25) (end 52.07 95.25) (width 0.25) (layer B.Cu) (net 1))
 (segment (start 89.884366 85.09) (end 85.09 89.884366) (width 0.25) (layer B.Cu) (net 1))
 (segment (start 73.66 107.95) (end 72.39 109.22) (width 0.25) (layer B.Cu) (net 1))
 (segment (start 85.09 89.884366) (end 85.09 100.33) (width 0.25) (layer B.Cu) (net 1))
 (segment (start 69.85 109.22) (end 67.31 106.68) (width 0.25) (layer B.Cu) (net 1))
 (segment (start 52.07 95.25) (end 49.53 97.79) (width 0.25) (layer B.Cu) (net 1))
 (segment (start 81.28 104.14) (end 74.93 104.14) (width 0.25) (layer B.Cu) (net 1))
 (segment (start 85.09 100.33) (end 81.28 104.14) (width 0.25) (layer B.Cu) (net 1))
 (segment (start 72.39 109.22) (end 69.85 109.22) (width 0.25) (layer B.Cu) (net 1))
 (segment (start 74.93 104.14) (end 73.66 105.41) (width 0.25) (layer B.Cu) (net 1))
 (segment (start 59.69 97.79) (end 59.69 96.52) (width 0.25) (layer B.Cu) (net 1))
 (segment (start 73.66 105.41) (end 73.66 107.95) (width 0.25) (layer B.Cu) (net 1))
 (segment (start 67.31 106.68) (end 67.31 105.41) (width 0.25) (layer B.Cu) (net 1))
 (segment (start 67.31 105.41) (end 59.69 97.79) (width 0.25) (layer B.Cu) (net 1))
 (segment (start 86.36 99.06) (end 91.44 104.14) (width 0.25) (layer F.Cu) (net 30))
 (segment (start 67.31 99.06) (end 86.36 99.06) (width 0.25) (layer F.Cu) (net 30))
 (segment (start 64.77 101.6) (end 67.31 99.06) (width 0.25) (layer F.Cu) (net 30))
 (segment (start 57.15 101.6) (end 64.77 101.6) (width 0.25) (layer F.Cu) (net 30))
 (segment (start 110.49 46.99) (end 105.41 46.99) (width 0.25) (layer B.Cu) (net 29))
 (segment (start 105.41 46.99) (end 102.87 49.53) (width 0.25) (layer B.Cu) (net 29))
 (segment (start 102.87 49.53) (end 102.87 109.22) (width 0.25) (layer B.Cu) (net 29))
 (segment (start 69.03001 109.67001) (end 64.77 105.41) (width 0.25) (layer B.Cu) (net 29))
 (segment (start 102.41999 109.67001) (end 69.03001 109.67001) (width 0.25) (layer B.Cu) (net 29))
 (segment (start 102.87 109.22) (end 102.41999 109.67001) (width 0.25) (layer B.Cu) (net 29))
 (segment (start 110.49 66.04) (end 106.68 66.04) (width 0.25) (layer B.Cu) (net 28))
 (segment (start 106.68 66.04) (end 104.14 68.58) (width 0.25) (layer B.Cu) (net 28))
 (segment (start 104.14 68.58) (end 104.14 109.22) (width 0.25) (layer B.Cu) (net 28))
 (segment (start 67.4964 111.30999) (end 62.86641 106.68) (width 0.25) (layer B.Cu) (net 28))
 (segment (start 102.05001 111.30999) (end 67.4964 111.30999) (width 0.25) (layer B.Cu) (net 28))
 (segment (start 104.14 109.22) (end 102.05001 111.30999) (width 0.25) (layer B.Cu) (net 28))
 (segment (start 62.86641 106.68) (end 54.61 106.68) (width 0.25) (layer B.Cu) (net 28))
 (segment (start 53.34 105.41) (end 49.53 105.41) (width 0.25) (layer B.Cu) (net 28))
 (segment (start 54.61 106.68) (end 53.34 105.41) (width 0.25) (layer B.Cu) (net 28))
 (segment (start 110.49 85.09) (end 107.95 85.09) (width 0.25) (layer B.Cu) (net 27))
 (segment (start 107.95 85.09) (end 105.41 87.63) (width 0.25) (layer B.Cu) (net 27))
 (segment (start 105.41 87.63) (end 105.41 109.22) (width 0.25) (layer B.Cu) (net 27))
 (segment (start 105.41 109.22) (end 102.87 111.76) (width 0.25) (layer B.Cu) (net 27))
 (segment (start 102.87 111.76) (end 67.31 111.76) (width 0.25) (layer B.Cu) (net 27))
 (segment (start 64.77 109.22) (end 57.15 109.22) (width 0.25) (layer B.Cu) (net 27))
 (segment (start 67.31 111.76) (end 64.77 109.22) (width 0.25) (layer B.Cu) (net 27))
 (segment (start 110.49 104.14) (end 107.95 104.14) (width 0.25) (layer B.Cu) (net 26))
 (segment (start 107.95 104.14) (end 106.68 105.41) (width 0.25) (layer B.Cu) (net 26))
 (segment (start 106.68 105.41) (end 106.68 109.22) (width 0.25) (layer B.Cu) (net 26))
 (segment (start 102.87 113.03) (end 64.77 113.03) (width 0.25) (layer B.Cu) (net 26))
 (segment (start 106.68 109.22) (end 102.87 113.03) (width 0.25) (layer B.Cu) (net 26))
 (segment (start 78.74 44.45) (end 78.74 101.6) (width 0.25) (layer B.Cu) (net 21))
 (segment (start 58.46 44.45) (end 43.22 59.69) (width 0.25) (layer B.Cu) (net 21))
 (segment (start 78.74 44.45) (end 58.46 44.45) (width 0.25) (layer B.Cu) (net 21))
 (segment (start 97.79 44.45) (end 97.79 101.6) (width 0.25) (layer B.Cu) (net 2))
 (segment (start 96.364999 43.024999) (end 40.795001 43.024999) (width 0.25) (layer F.Cu) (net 2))
 (segment (start 97.79 44.45) (end 96.364999 43.024999) (width 0.25) (layer F.Cu) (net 2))
 (segment (start 40.795001 43.024999) (end 39.37 44.45) (width 0.25) (layer F.Cu) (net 2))
 (segment (start 39.37 44.45) (end 39.37 60.96) (width 0.25) (layer F.Cu) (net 2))
 (segment (start 39.37 60.96) (end 40.64 62.23) (width 0.25) (layer F.Cu) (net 2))
 (segment (start 40.64 62.23) (end 43.22 62.23) (width 0.25) (layer F.Cu) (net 2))
 (segment (start 116.84 44.45) (end 116.84 101.6) (width 0.25) (layer B.Cu) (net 20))
 (segment (start 116.84 44.45) (end 114.3 41.91) (width 0.25) (layer B.Cu) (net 20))
 (segment (start 114.3 41.91) (end 45.72 41.91) (width 0.25) (layer B.Cu) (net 20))
 (segment (start 45.72 41.91) (end 39.37 48.26) (width 0.25) (layer B.Cu) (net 20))
 (segment (start 39.37 60.92) (end 43.22 64.77) (width 0.25) (layer B.Cu) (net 20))
 (segment (start 39.37 48.26) (end 39.37 60.92) (width 0.25) (layer B.Cu) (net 20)))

